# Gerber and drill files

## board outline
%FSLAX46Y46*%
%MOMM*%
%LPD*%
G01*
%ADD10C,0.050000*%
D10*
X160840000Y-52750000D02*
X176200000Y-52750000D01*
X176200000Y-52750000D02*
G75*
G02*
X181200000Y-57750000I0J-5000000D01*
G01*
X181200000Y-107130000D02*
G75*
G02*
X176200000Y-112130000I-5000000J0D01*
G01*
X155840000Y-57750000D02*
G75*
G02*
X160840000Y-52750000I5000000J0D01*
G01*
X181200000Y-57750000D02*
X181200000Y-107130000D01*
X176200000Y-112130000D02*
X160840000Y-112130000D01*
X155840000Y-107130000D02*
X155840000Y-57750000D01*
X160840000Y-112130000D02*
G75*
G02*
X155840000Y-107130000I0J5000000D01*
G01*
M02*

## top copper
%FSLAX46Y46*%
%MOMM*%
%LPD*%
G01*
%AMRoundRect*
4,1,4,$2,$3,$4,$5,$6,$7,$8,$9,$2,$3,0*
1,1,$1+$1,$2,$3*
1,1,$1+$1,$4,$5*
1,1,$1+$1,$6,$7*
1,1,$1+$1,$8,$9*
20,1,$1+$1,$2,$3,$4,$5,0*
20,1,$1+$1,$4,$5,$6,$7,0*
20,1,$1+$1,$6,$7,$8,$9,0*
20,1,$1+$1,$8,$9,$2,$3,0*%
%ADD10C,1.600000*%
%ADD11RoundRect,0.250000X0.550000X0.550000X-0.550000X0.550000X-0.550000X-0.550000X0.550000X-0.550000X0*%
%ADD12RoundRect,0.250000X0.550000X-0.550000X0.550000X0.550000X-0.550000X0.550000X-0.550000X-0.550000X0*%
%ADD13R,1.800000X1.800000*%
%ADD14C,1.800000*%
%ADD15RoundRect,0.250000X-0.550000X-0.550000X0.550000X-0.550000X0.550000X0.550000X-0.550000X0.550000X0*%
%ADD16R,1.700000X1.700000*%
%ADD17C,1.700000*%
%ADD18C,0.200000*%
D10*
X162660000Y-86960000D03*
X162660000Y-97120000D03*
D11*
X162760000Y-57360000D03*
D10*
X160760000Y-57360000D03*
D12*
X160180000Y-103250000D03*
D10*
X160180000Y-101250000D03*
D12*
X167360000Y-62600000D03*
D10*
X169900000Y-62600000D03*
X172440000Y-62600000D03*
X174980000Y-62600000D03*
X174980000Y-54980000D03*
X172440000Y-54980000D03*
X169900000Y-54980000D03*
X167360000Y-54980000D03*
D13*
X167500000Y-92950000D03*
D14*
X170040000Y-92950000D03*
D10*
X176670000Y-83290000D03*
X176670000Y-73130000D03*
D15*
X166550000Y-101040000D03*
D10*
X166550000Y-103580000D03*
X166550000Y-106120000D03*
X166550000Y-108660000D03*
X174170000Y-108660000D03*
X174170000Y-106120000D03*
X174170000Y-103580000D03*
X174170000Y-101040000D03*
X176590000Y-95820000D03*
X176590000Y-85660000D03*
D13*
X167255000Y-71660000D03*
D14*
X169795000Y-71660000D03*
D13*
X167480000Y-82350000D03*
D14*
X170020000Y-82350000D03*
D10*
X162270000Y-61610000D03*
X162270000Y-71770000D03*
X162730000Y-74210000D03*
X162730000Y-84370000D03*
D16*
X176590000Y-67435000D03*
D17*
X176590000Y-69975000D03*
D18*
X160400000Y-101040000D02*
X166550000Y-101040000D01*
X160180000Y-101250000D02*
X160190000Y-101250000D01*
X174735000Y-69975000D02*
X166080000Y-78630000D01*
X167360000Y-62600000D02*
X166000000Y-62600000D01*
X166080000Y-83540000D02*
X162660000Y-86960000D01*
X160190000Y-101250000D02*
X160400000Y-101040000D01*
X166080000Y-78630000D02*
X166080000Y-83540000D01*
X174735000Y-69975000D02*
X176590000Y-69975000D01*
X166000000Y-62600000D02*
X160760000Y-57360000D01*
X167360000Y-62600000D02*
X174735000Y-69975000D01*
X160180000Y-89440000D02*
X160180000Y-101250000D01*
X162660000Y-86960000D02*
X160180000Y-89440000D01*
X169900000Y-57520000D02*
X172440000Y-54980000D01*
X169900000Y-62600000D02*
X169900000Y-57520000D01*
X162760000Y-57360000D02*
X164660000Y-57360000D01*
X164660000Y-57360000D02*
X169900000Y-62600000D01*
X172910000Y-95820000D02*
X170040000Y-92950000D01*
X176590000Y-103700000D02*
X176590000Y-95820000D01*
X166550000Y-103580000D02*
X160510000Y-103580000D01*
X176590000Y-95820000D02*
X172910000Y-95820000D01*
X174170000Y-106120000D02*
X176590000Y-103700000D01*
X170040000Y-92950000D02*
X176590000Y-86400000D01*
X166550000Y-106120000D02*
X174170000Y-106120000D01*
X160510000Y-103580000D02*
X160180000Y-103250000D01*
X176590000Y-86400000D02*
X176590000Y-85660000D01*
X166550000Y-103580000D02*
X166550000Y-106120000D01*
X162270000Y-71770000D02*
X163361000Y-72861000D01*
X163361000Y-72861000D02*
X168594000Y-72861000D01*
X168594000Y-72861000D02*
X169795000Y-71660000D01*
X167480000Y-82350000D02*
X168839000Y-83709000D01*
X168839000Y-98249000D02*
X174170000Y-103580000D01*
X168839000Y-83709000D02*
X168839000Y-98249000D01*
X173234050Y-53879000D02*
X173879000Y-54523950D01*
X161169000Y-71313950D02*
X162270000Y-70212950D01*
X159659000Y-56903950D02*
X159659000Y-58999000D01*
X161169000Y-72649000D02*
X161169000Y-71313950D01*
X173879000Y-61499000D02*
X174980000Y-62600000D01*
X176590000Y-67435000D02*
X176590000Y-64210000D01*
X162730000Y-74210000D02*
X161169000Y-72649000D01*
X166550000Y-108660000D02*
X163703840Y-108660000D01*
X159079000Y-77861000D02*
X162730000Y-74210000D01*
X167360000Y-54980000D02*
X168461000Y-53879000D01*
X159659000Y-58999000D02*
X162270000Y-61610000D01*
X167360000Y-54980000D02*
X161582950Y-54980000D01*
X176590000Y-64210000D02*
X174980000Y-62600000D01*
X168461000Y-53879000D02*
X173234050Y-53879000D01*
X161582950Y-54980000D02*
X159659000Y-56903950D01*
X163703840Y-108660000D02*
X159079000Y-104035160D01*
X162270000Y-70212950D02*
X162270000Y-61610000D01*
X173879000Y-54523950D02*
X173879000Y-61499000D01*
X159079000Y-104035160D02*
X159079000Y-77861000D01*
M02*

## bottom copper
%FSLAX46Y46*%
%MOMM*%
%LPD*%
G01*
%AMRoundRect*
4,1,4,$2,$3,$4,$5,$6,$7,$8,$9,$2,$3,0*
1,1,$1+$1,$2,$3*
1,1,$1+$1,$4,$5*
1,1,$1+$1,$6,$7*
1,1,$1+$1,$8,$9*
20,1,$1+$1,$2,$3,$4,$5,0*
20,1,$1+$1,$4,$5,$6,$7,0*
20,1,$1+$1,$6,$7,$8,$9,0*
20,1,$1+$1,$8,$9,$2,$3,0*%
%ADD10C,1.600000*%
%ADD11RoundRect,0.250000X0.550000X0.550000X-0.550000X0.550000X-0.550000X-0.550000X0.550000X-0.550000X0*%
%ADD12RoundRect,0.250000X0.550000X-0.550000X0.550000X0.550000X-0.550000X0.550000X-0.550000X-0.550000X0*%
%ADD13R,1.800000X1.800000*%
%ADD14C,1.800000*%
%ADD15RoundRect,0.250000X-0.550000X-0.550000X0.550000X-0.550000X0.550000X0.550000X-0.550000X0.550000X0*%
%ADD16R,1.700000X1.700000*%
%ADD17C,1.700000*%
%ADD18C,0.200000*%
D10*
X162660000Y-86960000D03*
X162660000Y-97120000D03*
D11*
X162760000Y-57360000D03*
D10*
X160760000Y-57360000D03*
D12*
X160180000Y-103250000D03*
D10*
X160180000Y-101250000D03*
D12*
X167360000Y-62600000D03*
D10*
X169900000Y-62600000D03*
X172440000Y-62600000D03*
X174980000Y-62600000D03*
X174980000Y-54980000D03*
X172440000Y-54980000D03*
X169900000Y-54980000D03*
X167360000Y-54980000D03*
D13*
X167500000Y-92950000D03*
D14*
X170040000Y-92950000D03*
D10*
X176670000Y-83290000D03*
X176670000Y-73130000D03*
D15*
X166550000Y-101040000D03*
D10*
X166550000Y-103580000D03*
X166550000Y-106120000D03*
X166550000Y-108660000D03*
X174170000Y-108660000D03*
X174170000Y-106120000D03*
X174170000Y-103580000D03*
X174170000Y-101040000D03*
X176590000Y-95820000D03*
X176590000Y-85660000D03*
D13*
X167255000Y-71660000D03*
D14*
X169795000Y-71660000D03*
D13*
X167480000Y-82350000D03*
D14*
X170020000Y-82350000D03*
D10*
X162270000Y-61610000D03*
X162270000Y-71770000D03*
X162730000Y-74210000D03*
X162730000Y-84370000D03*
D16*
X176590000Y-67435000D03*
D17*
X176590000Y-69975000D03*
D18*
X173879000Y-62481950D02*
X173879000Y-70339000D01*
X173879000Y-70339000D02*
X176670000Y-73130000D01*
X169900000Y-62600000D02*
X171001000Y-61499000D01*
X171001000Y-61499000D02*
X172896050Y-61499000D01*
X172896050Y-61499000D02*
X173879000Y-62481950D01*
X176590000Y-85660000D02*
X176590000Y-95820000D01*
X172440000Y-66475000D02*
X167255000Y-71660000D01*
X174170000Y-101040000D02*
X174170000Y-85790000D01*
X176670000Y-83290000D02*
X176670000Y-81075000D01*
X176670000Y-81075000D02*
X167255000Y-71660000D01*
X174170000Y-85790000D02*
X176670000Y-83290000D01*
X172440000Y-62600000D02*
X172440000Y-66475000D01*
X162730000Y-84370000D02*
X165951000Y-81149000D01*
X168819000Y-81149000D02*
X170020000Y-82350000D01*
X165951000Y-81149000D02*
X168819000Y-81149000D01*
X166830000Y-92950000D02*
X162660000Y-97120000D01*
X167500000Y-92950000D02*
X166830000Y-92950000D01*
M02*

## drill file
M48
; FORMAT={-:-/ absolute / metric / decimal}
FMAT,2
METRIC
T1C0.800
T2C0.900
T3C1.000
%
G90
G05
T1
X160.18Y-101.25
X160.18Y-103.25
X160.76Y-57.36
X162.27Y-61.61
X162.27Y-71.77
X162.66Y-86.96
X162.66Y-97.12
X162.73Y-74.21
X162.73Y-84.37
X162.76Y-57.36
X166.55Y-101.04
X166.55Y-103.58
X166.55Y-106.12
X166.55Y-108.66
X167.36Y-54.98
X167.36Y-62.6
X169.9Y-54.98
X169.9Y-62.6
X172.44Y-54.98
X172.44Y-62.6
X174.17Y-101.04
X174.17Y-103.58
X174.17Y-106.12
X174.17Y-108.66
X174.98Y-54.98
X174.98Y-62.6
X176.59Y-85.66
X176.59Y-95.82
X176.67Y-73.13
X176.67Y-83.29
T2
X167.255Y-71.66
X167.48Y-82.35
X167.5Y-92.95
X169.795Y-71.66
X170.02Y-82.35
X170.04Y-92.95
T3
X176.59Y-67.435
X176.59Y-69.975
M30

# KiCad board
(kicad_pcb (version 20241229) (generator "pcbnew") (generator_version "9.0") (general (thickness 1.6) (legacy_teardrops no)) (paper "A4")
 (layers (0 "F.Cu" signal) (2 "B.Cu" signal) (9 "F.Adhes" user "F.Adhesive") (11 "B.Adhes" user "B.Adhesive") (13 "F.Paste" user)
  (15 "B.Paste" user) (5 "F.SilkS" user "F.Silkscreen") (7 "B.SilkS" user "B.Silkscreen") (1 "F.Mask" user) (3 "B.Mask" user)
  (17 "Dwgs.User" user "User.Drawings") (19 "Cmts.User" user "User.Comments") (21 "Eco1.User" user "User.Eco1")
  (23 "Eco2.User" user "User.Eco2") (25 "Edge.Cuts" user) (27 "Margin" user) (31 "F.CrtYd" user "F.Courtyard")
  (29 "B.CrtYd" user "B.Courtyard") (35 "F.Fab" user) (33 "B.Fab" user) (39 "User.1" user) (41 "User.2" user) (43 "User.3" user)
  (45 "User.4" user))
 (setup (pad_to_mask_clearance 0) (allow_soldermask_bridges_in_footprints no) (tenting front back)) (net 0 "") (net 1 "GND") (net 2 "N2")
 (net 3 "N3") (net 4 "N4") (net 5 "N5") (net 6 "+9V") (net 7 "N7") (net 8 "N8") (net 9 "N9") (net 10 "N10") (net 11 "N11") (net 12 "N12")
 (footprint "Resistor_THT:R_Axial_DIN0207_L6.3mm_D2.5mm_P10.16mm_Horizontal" (layer "F.Cu") (at 162.66 86.96 -90)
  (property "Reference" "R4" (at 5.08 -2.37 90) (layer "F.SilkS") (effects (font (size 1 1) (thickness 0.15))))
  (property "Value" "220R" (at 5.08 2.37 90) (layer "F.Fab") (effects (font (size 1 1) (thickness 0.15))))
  (pad "1" thru_hole circle (at 0 0 270) (size 1.6 1.6) (drill 0.8) (layers "*.Cu" "*.Mask") (remove_unused_layers no) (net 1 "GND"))
  (pad "2" thru_hole circle (at 10.16 0 270) (size 1.6 1.6) (drill 0.8) (layers "*.Cu" "*.Mask") (remove_unused_layers no) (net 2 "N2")))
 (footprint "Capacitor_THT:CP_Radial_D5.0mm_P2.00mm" (layer "F.Cu") (at 162.76 57.36 180)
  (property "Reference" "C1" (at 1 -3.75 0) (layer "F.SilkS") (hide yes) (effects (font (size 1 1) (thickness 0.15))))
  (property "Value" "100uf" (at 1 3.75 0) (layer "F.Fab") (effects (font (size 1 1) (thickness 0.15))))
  (pad "1" thru_hole roundrect (at 0 0 180) (size 1.6 1.6) (drill 0.8) (layers "*.Cu" "*.Mask") (remove_unused_layers no)
   (roundrect_rratio 0.15625) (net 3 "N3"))
  (pad "2" thru_hole circle (at 2 0 180) (size 1.6 1.6) (drill 0.8) (layers "*.Cu" "*.Mask") (remove_unused_layers no) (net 1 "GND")))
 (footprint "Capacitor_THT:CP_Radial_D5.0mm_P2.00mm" (layer "F.Cu") (at 160.18 103.25 90)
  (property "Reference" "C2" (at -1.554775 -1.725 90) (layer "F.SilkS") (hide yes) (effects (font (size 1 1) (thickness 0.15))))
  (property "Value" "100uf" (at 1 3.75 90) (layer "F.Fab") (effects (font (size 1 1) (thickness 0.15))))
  (pad "1" thru_hole roundrect (at 0 0 90) (size 1.6 1.6) (drill 0.8) (layers "*.Cu" "*.Mask") (remove_unused_layers no)
   (roundrect_rratio 0.15625) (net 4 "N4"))
  (pad "2" thru_hole circle (at 2 0 90) (size 1.6 1.6) (drill 0.8) (layers "*.Cu" "*.Mask") (remove_unused_layers no) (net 1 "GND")))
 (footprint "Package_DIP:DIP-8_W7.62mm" (layer "F.Cu") (at 167.36 62.6 90)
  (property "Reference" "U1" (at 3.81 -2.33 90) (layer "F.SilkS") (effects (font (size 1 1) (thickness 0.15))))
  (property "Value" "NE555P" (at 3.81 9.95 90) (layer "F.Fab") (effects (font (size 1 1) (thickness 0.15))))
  (pad "1" thru_hole roundrect (at 0 0 90) (size 1.6 1.6) (drill 0.8) (layers "*.Cu" "*.Mask") (remove_unused_layers no)
   (roundrect_rratio 0.15625) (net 1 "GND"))
  (pad "2" thru_hole circle (at 0 2.54 90) (size 1.6 1.6) (drill 0.8) (layers "*.Cu" "*.Mask") (remove_unused_layers no) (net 3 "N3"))
  (pad "3" thru_hole circle (at 0 5.08 90) (size 1.6 1.6) (drill 0.8) (layers "*.Cu" "*.Mask") (remove_unused_layers no) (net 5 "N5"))
  (pad "4" thru_hole circle (at 0 7.62 90) (size 1.6 1.6) (drill 0.8) (layers "*.Cu" "*.Mask") (remove_unused_layers no) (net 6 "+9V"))
  (pad "5" thru_hole circle (at 7.62 7.62 90) (size 1.6 1.6) (drill 0.8) (layers "*.Cu" "*.Mask") (remove_unused_layers no) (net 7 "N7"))
  (pad "6" thru_hole circle (at 7.62 5.08 90) (size 1.6 1.6) (drill 0.8) (layers "*.Cu" "*.Mask") (remove_unused_layers no) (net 3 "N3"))
  (pad "7" thru_hole circle (at 7.62 2.54 90) (size 1.6 1.6) (drill 0.8) (layers "*.Cu" "*.Mask") (remove_unused_layers no) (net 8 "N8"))
  (pad "8" thru_hole circle (at 7.62 0 90) (size 1.6 1.6) (drill 0.8) (layers "*.Cu" "*.Mask") (remove_unused_layers no) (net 6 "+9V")))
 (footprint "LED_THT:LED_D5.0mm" (layer "F.Cu") (at 167.5 92.95)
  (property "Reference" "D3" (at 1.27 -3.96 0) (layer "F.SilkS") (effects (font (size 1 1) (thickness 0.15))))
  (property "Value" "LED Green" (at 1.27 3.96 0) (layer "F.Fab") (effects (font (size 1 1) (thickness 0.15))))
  (pad "1" thru_hole rect (at 0 0) (size 1.8 1.8) (drill 0.9) (layers "*.Cu" "*.Mask") (remove_unused_layers no) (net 2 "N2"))
  (pad "2" thru_hole circle (at 2.54 0) (size 1.8 1.8) (drill 0.9) (layers "*.Cu" "*.Mask") (remove_unused_layers no) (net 4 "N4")))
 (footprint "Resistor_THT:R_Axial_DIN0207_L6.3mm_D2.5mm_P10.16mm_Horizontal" (layer "F.Cu") (at 176.67 83.29 90)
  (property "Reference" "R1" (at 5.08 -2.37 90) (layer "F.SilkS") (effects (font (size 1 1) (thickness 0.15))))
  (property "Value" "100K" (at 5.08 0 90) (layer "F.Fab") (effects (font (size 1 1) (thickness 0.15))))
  (pad "1" thru_hole circle (at 0 0 90) (size 1.6 1.6) (drill 0.8) (layers "*.Cu" "*.Mask") (remove_unused_layers no) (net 5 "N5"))
  (pad "2" thru_hole circle (at 10.16 0 90) (size 1.6 1.6) (drill 0.8) (layers "*.Cu" "*.Mask") (remove_unused_layers no) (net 3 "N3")))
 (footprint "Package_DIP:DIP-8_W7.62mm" (layer "F.Cu") (at 166.55 101.04)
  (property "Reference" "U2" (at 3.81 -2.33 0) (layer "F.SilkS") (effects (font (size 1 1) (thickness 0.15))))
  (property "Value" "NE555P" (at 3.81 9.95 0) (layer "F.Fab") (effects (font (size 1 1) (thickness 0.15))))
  (pad "1" thru_hole roundrect (at 0 0) (size 1.6 1.6) (drill 0.8) (layers "*.Cu" "*.Mask") (remove_unused_layers no)
   (roundrect_rratio 0.15625) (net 1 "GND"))
  (pad "2" thru_hole circle (at 0 2.54) (size 1.6 1.6) (drill 0.8) (layers "*.Cu" "*.Mask") (remove_unused_layers no) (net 4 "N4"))
  (pad "3" thru_hole circle (at 0 5.08) (size 1.6 1.6) (drill 0.8) (layers "*.Cu" "*.Mask") (remove_unused_layers no) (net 4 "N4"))
  (pad "4" thru_hole circle (at 0 7.62) (size 1.6 1.6) (drill 0.8) (layers "*.Cu" "*.Mask") (remove_unused_layers no) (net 6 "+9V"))
  (pad "5" thru_hole circle (at 7.62 7.62) (size 1.6 1.6) (drill 0.8) (layers "*.Cu" "*.Mask") (remove_unused_layers no) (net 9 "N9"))
  (pad "6" thru_hole circle (at 7.62 5.08) (size 1.6 1.6) (drill 0.8) (layers "*.Cu" "*.Mask") (remove_unused_layers no) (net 4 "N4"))
  (pad "7" thru_hole circle (at 7.62 2.54) (size 1.6 1.6) (drill 0.8) (layers "*.Cu" "*.Mask") (remove_unused_layers no) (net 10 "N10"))
  (pad "8" thru_hole circle (at 7.62 0) (size 1.6 1.6) (drill 0.8) (layers "*.Cu" "*.Mask") (remove_unused_layers no) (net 5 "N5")))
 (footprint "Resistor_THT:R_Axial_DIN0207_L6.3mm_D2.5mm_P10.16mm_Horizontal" (layer "F.Cu") (at 176.59 95.82 90)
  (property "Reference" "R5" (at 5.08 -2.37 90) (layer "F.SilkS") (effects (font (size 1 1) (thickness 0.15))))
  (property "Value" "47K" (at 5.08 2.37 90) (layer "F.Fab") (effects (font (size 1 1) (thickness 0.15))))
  (pad "1" thru_hole circle (at 0 0 90) (size 1.6 1.6) (drill 0.8) (layers "*.Cu" "*.Mask") (remove_unused_layers no) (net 4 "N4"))
  (pad "2" thru_hole circle (at 10.16 0 90) (size 1.6 1.6) (drill 0.8) (layers "*.Cu" "*.Mask") (remove_unused_layers no) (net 4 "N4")))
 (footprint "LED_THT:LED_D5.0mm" (layer "F.Cu") (at 167.255 71.66)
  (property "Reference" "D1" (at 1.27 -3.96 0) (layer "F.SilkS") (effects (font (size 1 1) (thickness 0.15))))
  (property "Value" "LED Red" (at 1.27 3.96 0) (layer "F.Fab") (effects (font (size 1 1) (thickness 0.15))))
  (pad "1" thru_hole rect (at 0 0) (size 1.8 1.8) (drill 0.9) (layers "*.Cu" "*.Mask") (remove_unused_layers no) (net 5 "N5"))
  (pad "2" thru_hole circle (at 2.54 0) (size 1.8 1.8) (drill 0.9) (layers "*.Cu" "*.Mask") (remove_unused_layers no) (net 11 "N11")))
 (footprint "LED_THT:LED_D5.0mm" (layer "F.Cu") (at 167.48 82.35)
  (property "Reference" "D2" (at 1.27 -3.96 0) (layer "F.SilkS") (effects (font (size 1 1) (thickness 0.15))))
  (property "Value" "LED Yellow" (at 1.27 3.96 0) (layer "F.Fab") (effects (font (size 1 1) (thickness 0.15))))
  (pad "1" thru_hole rect (at 0 0) (size 1.8 1.8) (drill 0.9) (layers "*.Cu" "*.Mask") (remove_unused_layers no) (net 10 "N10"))
  (pad "2" thru_hole circle (at 2.54 0) (size 1.8 1.8) (drill 0.9) (layers "*.Cu" "*.Mask") (remove_unused_layers no) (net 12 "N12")))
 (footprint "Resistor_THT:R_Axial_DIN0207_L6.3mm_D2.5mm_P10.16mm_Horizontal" (layer "F.Cu") (at 162.27 61.61 -90)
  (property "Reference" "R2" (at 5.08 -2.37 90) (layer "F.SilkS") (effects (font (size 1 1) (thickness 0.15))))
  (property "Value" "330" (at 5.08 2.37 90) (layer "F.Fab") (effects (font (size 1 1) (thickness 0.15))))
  (pad "1" thru_hole circle (at 0 0 270) (size 1.6 1.6) (drill 0.8) (layers "*.Cu" "*.Mask") (remove_unused_layers no) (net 6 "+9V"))
  (pad "2" thru_hole circle (at 10.16 0 270) (size 1.6 1.6) (drill 0.8) (layers "*.Cu" "*.Mask") (remove_unused_layers no) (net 11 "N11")))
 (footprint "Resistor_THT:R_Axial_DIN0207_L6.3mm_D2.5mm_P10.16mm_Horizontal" (layer "F.Cu") (at 162.73 74.21 -90)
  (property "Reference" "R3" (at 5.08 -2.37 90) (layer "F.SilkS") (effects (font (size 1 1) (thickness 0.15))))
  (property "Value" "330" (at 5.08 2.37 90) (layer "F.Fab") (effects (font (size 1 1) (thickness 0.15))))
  (pad "1" thru_hole circle (at 0 0 270) (size 1.6 1.6) (drill 0.8) (layers "*.Cu" "*.Mask") (remove_unused_layers no) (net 6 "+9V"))
  (pad "2" thru_hole circle (at 10.16 0 270) (size 1.6 1.6) (drill 0.8) (layers "*.Cu" "*.Mask") (remove_unused_layers no) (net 12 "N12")))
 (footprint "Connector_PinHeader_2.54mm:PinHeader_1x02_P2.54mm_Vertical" (layer "F.Cu") (at 176.59 67.435)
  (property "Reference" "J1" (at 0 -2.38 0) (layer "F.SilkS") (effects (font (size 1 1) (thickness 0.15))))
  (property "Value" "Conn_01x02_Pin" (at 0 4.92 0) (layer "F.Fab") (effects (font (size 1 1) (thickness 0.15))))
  (pad "1" thru_hole rect (at 0 0) (size 1.7 1.7) (drill 1) (layers "*.Cu" "*.Mask") (remove_unused_layers no) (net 6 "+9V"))
  (pad "2" thru_hole circle (at 0 2.54) (size 1.7 1.7) (drill 1) (layers "*.Cu" "*.Mask") (remove_unused_layers no) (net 1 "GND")))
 (gr_line (start 160.84 52.75) (end 176.2 52.75) (stroke (width 0.05) (type default)) (layer "Edge.Cuts"))
 (gr_arc (start 176.2 52.75) (mid 179.735534 54.214466) (end 181.2 57.75) (stroke (width 0.05) (type default)) (layer "Edge.Cuts"))
 (gr_arc (start 181.2 107.13) (mid 179.735534 110.665534) (end 176.2 112.13) (stroke (width 0.05) (type default)) (layer "Edge.Cuts"))
 (gr_arc (start 155.84 57.75) (mid 157.304466 54.214466) (end 160.84 52.75) (stroke (width 0.05) (type default)) (layer "Edge.Cuts"))
 (gr_line (start 181.2 57.75) (end 181.2 107.13) (stroke (width 0.05) (type default)) (layer "Edge.Cuts"))
 (gr_line (start 176.2 112.13) (end 160.84 112.13) (stroke (width 0.05) (type default)) (layer "Edge.Cuts"))
 (gr_line (start 155.84 107.13) (end 155.84 57.75) (stroke (width 0.05) (type default)) (layer "Edge.Cuts"))
 (gr_arc (start 160.84 112.13) (mid 157.304466 110.665534) (end 155.84 107.13) (stroke (width 0.05) (type default)) (layer "Edge.Cuts"))
 (segment (start 160.4 101.04) (end 166.55 101.04) (width 0.2) (layer "F.Cu") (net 1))
 (segment (start 160.18 101.25) (end 160.19 101.25) (width 0.2) (layer "F.Cu") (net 1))
 (segment (start 174.735 69.975) (end 166.08 78.63) (width 0.2) (layer "F.Cu") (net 1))
 (segment (start 167.36 62.6) (end 166 62.6) (width 0.2) (layer "F.Cu") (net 1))
 (segment (start 166.08 83.54) (end 162.66 86.96) (width 0.2) (layer "F.Cu") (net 1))
 (segment (start 160.19 101.25) (end 160.4 101.04) (width 0.2) (layer "F.Cu") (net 1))
 (segment (start 166.08 78.63) (end 166.08 83.54) (width 0.2) (layer "F.Cu") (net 1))
 (segment (start 174.735 69.975) (end 176.59 69.975) (width 0.2) (layer "F.Cu") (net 1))
 (segment (start 166 62.6) (end 160.76 57.36) (width 0.2) (layer "F.Cu") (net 1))
 (segment (start 167.36 62.6) (end 174.735 69.975) (width 0.2) (layer "F.Cu") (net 1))
 (segment (start 160.18 89.44) (end 160.18 101.25) (width 0.2) (layer "F.Cu") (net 1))
 (segment (start 162.66 86.96) (end 160.18 89.44) (width 0.2) (layer "F.Cu") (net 1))
 (segment (start 169.9 57.52) (end 172.44 54.98) (width 0.2) (layer "F.Cu") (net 3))
 (segment (start 169.9 62.6) (end 169.9 57.52) (width 0.2) (layer "F.Cu") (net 3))
 (segment (start 162.76 57.36) (end 164.66 57.36) (width 0.2) (layer "F.Cu") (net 3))
 (segment (start 164.66 57.36) (end 169.9 62.6) (width 0.2) (layer "F.Cu") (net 3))
 (segment (start 173.879 62.48195) (end 173.879 70.339) (width 0.2) (layer "B.Cu") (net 3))
 (segment (start 173.879 70.339) (end 176.67 73.13) (width 0.2) (layer "B.Cu") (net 3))
 (segment (start 169.9 62.6) (end 171.001 61.499) (width 0.2) (layer "B.Cu") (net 3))
 (segment (start 171.001 61.499) (end 172.89605 61.499) (width 0.2) (layer "B.Cu") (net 3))
 (segment (start 172.89605 61.499) (end 173.879 62.48195) (width 0.2) (layer "B.Cu") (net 3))
 (segment (start 172.91 95.82) (end 170.04 92.95) (width 0.2) (layer "F.Cu") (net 4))
 (segment (start 176.59 103.7) (end 176.59 95.82) (width 0.2) (layer "F.Cu") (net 4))
 (segment (start 166.55 103.58) (end 160.51 103.58) (width 0.2) (layer "F.Cu") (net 4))
 (segment (start 176.59 95.82) (end 172.91 95.82) (width 0.2) (layer "F.Cu") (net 4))
 (segment (start 174.17 106.12) (end 176.59 103.7) (width 0.2) (layer "F.Cu") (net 4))
 (segment (start 170.04 92.95) (end 176.59 86.4) (width 0.2) (layer "F.Cu") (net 4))
 (segment (start 166.55 106.12) (end 174.17 106.12) (width 0.2) (layer "F.Cu") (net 4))
 (segment (start 160.51 103.58) (end 160.18 103.25) (width 0.2) (layer "F.Cu") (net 4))
 (segment (start 176.59 86.4) (end 176.59 85.66) (width 0.2) (layer "F.Cu") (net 4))
 (segment (start 166.55 103.58) (end 166.55 106.12) (width 0.2) (layer "F.Cu") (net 4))
 (segment (start 176.59 85.66) (end 176.59 95.82) (width 0.2) (layer "B.Cu") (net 4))
 (segment (start 162.27 71.77) (end 163.361 72.861) (width 0.2) (layer "F.Cu") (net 11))
 (segment (start 163.361 72.861) (end 168.594 72.861) (width 0.2) (layer "F.Cu") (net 11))
 (segment (start 168.594 72.861) (end 169.795 71.66) (width 0.2) (layer "F.Cu") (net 11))
 (segment (start 172.44 66.475) (end 167.255 71.66) (width 0.2) (layer "B.Cu") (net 5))
 (segment (start 174.17 101.04) (end 174.17 85.79) (width 0.2) (layer "B.Cu") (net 5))
 (segment (start 176.67 83.29) (end 176.67 81.075) (width 0.2) (layer "B.Cu") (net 5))
 (segment (start 176.67 81.075) (end 167.255 71.66) (width 0.2) (layer "B.Cu") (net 5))
 (segment (start 174.17 85.79) (end 176.67 83.29) (width 0.2) (layer "B.Cu") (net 5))
 (segment (start 172.44 62.6) (end 172.44 66.475) (width 0.2) (layer "B.Cu") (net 5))
 (segment (start 167.48 82.35) (end 168.839 83.709) (width 0.2) (layer "F.Cu") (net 10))
 (segment (start 168.839 98.249) (end 174.17 103.58) (width 0.2) (layer "F.Cu") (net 10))
 (segment (start 168.839 83.709) (end 168.839 98.249) (width 0.2) (layer "F.Cu") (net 10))
 (segment (start 162.73 84.37) (end 165.951 81.149) (width 0.2) (layer "B.Cu") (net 12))
 (segment (start 168.819 81.149) (end 170.02 82.35) (width 0.2) (layer "B.Cu") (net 12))
 (segment (start 165.951 81.149) (end 168.819 81.149) (width 0.2) (layer "B.Cu") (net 12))
 (segment (start 166.83 92.95) (end 162.66 97.12) (width 0.2) (layer "B.Cu") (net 2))
 (segment (start 167.5 92.95) (end 166.83 92.95) (width 0.2) (layer "B.Cu") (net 2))
 (segment (start 173.23405 53.879) (end 173.879 54.52395) (width 0.2) (layer "F.Cu") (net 6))
 (segment (start 161.169 71.31395) (end 162.27 70.21295) (width 0.2) (layer "F.Cu") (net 6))
 (segment (start 159.659 56.90395) (end 159.659 58.999) (width 0.2) (layer "F.Cu") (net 6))
 (segment (start 161.169 72.649) (end 161.169 71.31395) (width 0.2) (layer "F.Cu") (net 6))
 (segment (start 173.879 61.499) (end 174.98 62.6) (width 0.2) (layer "F.Cu") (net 6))
 (segment (start 176.59 67.435) (end 176.59 64.21) (width 0.2) (layer "F.Cu") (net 6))
 (segment (start 162.73 74.21) (end 161.169 72.649) (width 0.2) (layer "F.Cu") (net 6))
 (segment (start 166.55 108.66) (end 163.70384 108.66) (width 0.2) (layer "F.Cu") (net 6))
 (segment (start 159.079 77.861) (end 162.73 74.21) (width 0.2) (layer "F.Cu") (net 6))
 (segment (start 167.36 54.98) (end 168.461 53.879) (width 0.2) (layer "F.Cu") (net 6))
 (segment (start 159.659 58.999) (end 162.27 61.61) (width 0.2) (layer "F.Cu") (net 6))
 (segment (start 167.36 54.98) (end 161.58295 54.98) (width 0.2) (layer "F.Cu") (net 6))
 (segment (start 176.59 64.21) (end 174.98 62.6) (width 0.2) (layer "F.Cu") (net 6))
 (segment (start 168.461 53.879) (end 173.23405 53.879) (width 0.2) (layer "F.Cu") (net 6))
 (segment (start 161.58295 54.98) (end 159.659 56.90395) (width 0.2) (layer "F.Cu") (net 6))
 (segment (start 163.70384 108.66) (end 159.079 104.03516) (width 0.2) (layer "F.Cu") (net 6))
 (segment (start 162.27 70.21295) (end 162.27 61.61) (width 0.2) (layer "F.Cu") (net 6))
 (segment (start 173.879 54.52395) (end 173.879 61.499) (width 0.2) (layer "F.Cu") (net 6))
 (segment (start 159.079 104.03516) (end 159.079 77.861) (width 0.2) (layer "F.Cu") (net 6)))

